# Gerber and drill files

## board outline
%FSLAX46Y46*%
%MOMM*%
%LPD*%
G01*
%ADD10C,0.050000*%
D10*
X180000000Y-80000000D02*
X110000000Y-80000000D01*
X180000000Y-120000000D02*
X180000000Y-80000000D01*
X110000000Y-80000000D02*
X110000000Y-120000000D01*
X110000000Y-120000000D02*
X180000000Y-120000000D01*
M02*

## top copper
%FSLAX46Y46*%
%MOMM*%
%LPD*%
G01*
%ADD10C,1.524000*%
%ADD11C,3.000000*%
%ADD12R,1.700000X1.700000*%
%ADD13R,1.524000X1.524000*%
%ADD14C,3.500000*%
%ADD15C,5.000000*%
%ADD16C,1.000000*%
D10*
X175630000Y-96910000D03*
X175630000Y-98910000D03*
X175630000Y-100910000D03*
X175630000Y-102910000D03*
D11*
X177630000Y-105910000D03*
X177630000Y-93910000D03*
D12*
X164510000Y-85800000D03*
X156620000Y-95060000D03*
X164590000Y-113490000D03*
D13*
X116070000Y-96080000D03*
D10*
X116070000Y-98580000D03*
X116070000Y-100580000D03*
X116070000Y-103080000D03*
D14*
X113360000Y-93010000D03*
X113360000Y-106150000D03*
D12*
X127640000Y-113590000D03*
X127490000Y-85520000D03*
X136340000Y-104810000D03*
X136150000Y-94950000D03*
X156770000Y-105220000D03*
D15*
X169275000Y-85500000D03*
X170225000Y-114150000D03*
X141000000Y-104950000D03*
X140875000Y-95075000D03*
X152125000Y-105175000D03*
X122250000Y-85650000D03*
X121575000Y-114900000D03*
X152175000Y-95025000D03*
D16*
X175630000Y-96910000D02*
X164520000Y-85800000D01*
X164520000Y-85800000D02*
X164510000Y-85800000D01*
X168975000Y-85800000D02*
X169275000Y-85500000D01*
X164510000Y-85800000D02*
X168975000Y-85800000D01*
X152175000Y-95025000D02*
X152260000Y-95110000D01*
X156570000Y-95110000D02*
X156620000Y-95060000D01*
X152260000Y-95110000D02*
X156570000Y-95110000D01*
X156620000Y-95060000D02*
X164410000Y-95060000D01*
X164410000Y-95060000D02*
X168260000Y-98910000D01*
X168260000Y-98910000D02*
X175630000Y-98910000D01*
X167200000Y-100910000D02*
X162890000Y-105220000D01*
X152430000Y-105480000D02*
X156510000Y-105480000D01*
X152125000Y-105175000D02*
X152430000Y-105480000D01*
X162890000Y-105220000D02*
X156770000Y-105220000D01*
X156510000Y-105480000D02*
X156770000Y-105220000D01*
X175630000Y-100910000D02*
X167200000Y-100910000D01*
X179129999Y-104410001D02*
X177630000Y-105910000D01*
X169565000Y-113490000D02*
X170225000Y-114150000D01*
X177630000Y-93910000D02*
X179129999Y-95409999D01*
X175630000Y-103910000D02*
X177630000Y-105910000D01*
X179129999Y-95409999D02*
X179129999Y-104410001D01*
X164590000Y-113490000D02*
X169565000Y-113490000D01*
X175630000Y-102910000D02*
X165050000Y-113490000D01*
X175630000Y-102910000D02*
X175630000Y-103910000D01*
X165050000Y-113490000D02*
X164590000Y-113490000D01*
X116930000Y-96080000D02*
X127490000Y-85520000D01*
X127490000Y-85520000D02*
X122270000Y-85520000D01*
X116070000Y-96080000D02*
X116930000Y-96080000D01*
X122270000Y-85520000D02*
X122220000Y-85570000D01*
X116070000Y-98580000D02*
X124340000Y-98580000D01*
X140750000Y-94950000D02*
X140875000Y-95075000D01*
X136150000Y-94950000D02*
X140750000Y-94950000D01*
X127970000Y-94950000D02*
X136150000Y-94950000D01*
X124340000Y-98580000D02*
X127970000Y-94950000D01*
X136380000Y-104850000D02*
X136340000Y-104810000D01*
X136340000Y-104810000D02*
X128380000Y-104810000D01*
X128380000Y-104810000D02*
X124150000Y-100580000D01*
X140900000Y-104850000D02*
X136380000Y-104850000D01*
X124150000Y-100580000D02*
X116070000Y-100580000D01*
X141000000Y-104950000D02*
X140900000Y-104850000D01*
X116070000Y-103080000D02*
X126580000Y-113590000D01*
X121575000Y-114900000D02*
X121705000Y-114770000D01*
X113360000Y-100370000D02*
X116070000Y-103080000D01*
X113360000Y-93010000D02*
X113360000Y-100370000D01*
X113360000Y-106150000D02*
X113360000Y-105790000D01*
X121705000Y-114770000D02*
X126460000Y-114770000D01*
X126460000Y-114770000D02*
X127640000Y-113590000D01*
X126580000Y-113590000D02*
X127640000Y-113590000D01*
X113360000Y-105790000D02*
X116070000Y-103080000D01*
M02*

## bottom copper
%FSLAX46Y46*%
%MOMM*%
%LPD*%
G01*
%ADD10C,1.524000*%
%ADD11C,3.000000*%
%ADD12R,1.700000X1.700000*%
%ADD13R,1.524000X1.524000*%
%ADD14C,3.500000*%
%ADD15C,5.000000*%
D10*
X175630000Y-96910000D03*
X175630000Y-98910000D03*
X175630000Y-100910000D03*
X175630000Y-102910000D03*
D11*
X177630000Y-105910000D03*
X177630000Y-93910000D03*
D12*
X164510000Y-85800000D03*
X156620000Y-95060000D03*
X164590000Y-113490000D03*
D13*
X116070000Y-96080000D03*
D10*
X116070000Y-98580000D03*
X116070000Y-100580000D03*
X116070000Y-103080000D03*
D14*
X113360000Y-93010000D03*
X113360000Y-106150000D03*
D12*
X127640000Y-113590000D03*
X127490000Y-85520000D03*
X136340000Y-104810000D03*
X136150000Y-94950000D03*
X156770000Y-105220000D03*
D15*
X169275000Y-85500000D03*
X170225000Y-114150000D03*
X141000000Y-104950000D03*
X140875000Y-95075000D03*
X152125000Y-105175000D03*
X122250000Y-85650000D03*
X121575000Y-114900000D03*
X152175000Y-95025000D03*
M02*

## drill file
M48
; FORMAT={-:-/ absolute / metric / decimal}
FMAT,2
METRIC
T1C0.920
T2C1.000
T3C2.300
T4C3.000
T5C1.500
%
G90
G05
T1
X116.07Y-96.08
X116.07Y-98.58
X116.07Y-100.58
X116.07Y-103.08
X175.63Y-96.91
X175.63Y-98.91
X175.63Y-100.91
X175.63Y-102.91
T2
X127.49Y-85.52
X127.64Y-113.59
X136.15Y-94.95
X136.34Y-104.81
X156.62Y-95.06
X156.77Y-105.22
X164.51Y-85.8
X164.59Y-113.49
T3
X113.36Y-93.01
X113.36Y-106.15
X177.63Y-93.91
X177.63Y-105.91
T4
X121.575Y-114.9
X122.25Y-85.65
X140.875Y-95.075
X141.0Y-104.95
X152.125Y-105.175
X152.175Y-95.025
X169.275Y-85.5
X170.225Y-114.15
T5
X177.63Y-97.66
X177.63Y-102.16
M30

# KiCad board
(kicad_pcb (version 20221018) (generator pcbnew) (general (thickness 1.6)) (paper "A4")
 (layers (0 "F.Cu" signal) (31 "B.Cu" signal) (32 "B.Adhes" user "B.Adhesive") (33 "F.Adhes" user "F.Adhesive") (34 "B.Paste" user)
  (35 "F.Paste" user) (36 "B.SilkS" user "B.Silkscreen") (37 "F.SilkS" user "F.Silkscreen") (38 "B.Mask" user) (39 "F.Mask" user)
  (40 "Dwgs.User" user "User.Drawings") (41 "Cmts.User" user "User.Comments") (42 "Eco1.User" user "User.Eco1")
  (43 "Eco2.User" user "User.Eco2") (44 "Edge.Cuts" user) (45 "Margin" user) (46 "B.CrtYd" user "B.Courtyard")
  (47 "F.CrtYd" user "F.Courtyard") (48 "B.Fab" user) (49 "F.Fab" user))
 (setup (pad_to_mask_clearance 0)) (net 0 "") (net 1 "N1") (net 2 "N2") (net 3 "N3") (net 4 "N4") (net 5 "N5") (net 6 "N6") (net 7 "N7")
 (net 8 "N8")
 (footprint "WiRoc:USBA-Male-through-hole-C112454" (layer "F.Cu") (at 177.63 99.91 90)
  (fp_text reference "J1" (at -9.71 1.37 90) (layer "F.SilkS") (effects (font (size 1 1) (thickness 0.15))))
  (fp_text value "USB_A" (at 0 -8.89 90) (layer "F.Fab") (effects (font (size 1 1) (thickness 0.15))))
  (pad "" np_thru_hole circle (at -2.25 0 90) (size 1.5 1.5) (drill 1.5) (layers "*.Cu" "*.Mask"))
  (pad "" np_thru_hole circle (at 2.25 0 90) (size 1.5 1.5) (drill 1.5) (layers "*.Cu" "*.Mask"))
  (pad "1" thru_hole circle (at 3 -2 90) (size 1.524 1.524) (drill 0.92) (layers "*.Cu" "*.Mask") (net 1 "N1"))
  (pad "2" thru_hole circle (at 1 -2 90) (size 1.524 1.524) (drill 0.92) (layers "*.Cu" "*.Mask") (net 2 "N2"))
  (pad "3" thru_hole circle (at -1 -2 90) (size 1.524 1.524) (drill 0.92) (layers "*.Cu" "*.Mask") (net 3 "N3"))
  (pad "4" thru_hole circle (at -3 -2 90) (size 1.524 1.524) (drill 0.92) (layers "*.Cu" "*.Mask") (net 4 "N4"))
  (pad "5" thru_hole circle (at -6 0 90) (size 3 3) (drill 2.3) (layers "*.Cu" "*.Mask") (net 4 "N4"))
  (pad "5" thru_hole circle (at 6 0 90) (size 3 3) (drill 2.3) (layers "*.Cu" "*.Mask") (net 4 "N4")))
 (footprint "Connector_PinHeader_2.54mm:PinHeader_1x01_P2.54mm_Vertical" (layer "F.Cu") (at 164.51 85.8 90)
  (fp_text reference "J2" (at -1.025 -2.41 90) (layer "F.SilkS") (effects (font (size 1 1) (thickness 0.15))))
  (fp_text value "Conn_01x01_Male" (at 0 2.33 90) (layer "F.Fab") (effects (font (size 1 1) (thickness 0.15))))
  (pad "1" thru_hole rect (at 0 0 90) (size 1.7 1.7) (drill 1) (layers "*.Cu" "*.Mask") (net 1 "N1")))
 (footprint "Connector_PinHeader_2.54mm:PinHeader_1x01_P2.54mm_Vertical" (layer "F.Cu") (at 156.62 95.06 90)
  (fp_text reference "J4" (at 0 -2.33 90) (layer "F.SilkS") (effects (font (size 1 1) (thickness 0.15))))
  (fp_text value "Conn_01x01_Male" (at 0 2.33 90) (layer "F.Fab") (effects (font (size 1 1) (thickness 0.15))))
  (pad "1" thru_hole rect (at 0 0 90) (size 1.7 1.7) (drill 1) (layers "*.Cu" "*.Mask") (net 2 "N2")))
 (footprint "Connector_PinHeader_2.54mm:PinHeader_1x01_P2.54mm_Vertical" (layer "F.Cu") (at 164.59 113.49 90)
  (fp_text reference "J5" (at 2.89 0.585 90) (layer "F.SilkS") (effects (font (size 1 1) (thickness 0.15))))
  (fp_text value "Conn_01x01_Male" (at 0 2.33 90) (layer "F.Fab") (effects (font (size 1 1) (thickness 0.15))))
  (pad "1" thru_hole rect (at 0 0 90) (size 1.7 1.7) (drill 1) (layers "*.Cu" "*.Mask") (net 4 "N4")))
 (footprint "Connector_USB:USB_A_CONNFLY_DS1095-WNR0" (layer "F.Cu") (at 116.07 96.08 -90)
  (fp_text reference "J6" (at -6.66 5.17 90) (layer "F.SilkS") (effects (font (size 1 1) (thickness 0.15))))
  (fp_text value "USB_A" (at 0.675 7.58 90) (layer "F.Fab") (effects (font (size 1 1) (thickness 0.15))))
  (pad "1" thru_hole rect (at 0 0 270) (size 1.524 1.524) (drill 0.92) (layers "*.Cu" "*.Mask") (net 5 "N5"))
  (pad "2" thru_hole circle (at 2.5 0 270) (size 1.524 1.524) (drill 0.92) (layers "*.Cu" "*.Mask") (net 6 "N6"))
  (pad "3" thru_hole circle (at 4.5 0 270) (size 1.524 1.524) (drill 0.92) (layers "*.Cu" "*.Mask") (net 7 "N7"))
  (pad "4" thru_hole circle (at 7 0 270) (size 1.524 1.524) (drill 0.92) (layers "*.Cu" "*.Mask") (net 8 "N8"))
  (pad "5" thru_hole circle (at -3.07 2.71 270) (size 3.5 3.5) (drill 2.3) (layers "*.Cu" "*.Mask") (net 8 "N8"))
  (pad "5" thru_hole circle (at 10.07 2.71 270) (size 3.5 3.5) (drill 2.3) (layers "*.Cu" "*.Mask") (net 8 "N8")))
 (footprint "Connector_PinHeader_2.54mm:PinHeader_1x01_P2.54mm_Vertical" (layer "F.Cu") (at 127.64 113.59 90)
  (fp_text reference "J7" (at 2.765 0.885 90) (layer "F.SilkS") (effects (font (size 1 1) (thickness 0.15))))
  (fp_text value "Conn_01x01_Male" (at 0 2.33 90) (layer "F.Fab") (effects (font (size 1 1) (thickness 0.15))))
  (pad "1" thru_hole rect (at 0 0 90) (size 1.7 1.7) (drill 1) (layers "*.Cu" "*.Mask") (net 8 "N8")))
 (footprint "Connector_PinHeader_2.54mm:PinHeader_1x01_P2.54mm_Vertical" (layer "F.Cu") (at 127.49 85.52 90)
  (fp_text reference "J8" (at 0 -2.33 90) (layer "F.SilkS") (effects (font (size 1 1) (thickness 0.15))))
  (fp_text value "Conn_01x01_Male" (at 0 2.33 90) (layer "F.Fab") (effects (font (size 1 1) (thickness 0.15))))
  (pad "1" thru_hole rect (at 0 0 90) (size 1.7 1.7) (drill 1) (layers "*.Cu" "*.Mask") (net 5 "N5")))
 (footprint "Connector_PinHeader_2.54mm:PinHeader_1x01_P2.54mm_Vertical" (layer "F.Cu") (at 136.34 104.81 90)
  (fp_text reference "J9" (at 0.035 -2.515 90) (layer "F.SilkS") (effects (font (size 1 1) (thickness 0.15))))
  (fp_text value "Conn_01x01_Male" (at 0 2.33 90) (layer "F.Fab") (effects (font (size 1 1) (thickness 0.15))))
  (pad "1" thru_hole rect (at 0 0 90) (size 1.7 1.7) (drill 1) (layers "*.Cu" "*.Mask") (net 7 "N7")))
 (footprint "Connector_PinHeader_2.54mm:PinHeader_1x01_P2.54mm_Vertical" (layer "F.Cu") (at 136.15 94.95 90)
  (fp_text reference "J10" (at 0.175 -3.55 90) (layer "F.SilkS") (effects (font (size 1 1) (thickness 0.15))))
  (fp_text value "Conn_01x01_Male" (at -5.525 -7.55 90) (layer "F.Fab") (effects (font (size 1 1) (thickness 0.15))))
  (pad "1" thru_hole rect (at 0 0 90) (size 1.7 1.7) (drill 1) (layers "*.Cu" "*.Mask") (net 6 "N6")))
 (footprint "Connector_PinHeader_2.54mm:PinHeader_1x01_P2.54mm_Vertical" (layer "F.Cu") (at 156.77 105.22 90)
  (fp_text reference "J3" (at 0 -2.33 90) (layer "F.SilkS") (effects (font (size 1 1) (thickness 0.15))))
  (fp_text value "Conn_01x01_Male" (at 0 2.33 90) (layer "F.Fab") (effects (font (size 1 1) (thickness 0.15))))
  (pad "1" thru_hole rect (at 0 0 90) (size 1.7 1.7) (drill 1) (layers "*.Cu" "*.Mask") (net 3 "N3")))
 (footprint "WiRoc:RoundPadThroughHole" (layer "F.Cu") (at 169.275 85.5)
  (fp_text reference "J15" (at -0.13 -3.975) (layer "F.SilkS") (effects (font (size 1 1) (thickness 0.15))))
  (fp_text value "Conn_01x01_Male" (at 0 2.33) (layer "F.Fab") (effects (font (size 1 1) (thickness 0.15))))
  (pad "1" thru_hole circle (at 0 0) (size 5 5) (drill 3) (layers "*.Cu" "*.Mask") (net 1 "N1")))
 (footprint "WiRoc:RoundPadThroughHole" (layer "F.Cu") (at 170.225 114.15)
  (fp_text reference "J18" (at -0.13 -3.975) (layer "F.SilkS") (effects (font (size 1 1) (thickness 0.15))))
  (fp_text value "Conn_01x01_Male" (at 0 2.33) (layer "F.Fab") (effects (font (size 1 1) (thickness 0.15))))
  (pad "1" thru_hole circle (at 0 0) (size 5 5) (drill 3) (layers "*.Cu" "*.Mask") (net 4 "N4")))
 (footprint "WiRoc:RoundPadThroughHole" (layer "F.Cu") (at 141 104.95)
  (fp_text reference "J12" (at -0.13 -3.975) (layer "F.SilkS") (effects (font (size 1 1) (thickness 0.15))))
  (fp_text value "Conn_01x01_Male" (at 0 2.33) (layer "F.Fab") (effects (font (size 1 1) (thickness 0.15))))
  (pad "1" thru_hole circle (at 0 0) (size 5 5) (drill 3) (layers "*.Cu" "*.Mask") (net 7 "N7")))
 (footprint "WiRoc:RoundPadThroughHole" (layer "F.Cu") (at 140.875 95.075)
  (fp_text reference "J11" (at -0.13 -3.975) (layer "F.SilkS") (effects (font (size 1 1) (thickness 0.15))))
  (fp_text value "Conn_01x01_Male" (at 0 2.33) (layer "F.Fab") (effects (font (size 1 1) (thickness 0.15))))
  (pad "1" thru_hole circle (at 0 0) (size 5 5) (drill 3) (layers "*.Cu" "*.Mask") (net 6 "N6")))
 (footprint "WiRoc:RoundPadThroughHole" (layer "F.Cu") (at 152.125 105.175)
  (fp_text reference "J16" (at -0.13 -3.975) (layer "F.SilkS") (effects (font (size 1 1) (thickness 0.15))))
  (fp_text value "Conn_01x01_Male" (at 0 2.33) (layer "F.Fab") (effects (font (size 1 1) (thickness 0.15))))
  (pad "1" thru_hole circle (at 0 0) (size 5 5) (drill 3) (layers "*.Cu" "*.Mask") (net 3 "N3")))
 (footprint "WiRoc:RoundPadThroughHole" (layer "F.Cu") (at 122.25 85.65)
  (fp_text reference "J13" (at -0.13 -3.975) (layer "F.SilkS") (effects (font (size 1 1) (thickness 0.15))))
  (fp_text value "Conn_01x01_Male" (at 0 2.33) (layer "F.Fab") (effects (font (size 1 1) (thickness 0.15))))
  (pad "1" thru_hole circle (at 0 0) (size 5 5) (drill 3) (layers "*.Cu" "*.Mask") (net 5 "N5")))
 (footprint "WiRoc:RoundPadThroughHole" (layer "F.Cu") (at 121.575 114.9)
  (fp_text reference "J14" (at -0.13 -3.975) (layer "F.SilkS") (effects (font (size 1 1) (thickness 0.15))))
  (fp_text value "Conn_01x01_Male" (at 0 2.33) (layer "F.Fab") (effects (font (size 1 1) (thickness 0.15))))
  (pad "1" thru_hole circle (at 0 0) (size 5 5) (drill 3) (layers "*.Cu" "*.Mask") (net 8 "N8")))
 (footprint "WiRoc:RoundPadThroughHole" (layer "F.Cu") (at 152.175 95.025)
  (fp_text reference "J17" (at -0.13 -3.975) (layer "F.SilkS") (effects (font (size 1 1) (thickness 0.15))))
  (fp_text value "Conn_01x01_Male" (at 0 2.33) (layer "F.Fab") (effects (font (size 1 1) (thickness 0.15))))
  (pad "1" thru_hole circle (at 0 0) (size 5 5) (drill 3) (layers "*.Cu" "*.Mask") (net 2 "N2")))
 (gr_line (start 180 80) (end 110 80) (stroke (width 0.05) (type solid)) (layer "Edge.Cuts"))
 (gr_line (start 180 120) (end 180 80) (stroke (width 0.05) (type solid)) (layer "Edge.Cuts"))
 (gr_line (start 110 80) (end 110 120) (stroke (width 0.05) (type solid)) (layer "Edge.Cuts"))
 (gr_line (start 110 120) (end 180 120) (stroke (width 0.05) (type solid)) (layer "Edge.Cuts"))
 (segment (start 175.63 96.91) (end 164.52 85.8) (width 1) (layer "F.Cu") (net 1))
 (segment (start 164.52 85.8) (end 164.51 85.8) (width 1) (layer "F.Cu") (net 1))
 (segment (start 168.975 85.8) (end 169.275 85.5) (width 1) (layer "F.Cu") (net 1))
 (segment (start 164.51 85.8) (end 168.975 85.8) (width 1) (layer "F.Cu") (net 1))
 (segment (start 152.175 95.025) (end 152.26 95.11) (width 1) (layer "F.Cu") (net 2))
 (segment (start 156.57 95.11) (end 156.62 95.06) (width 1) (layer "F.Cu") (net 2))
 (segment (start 152.26 95.11) (end 156.57 95.11) (width 1) (layer "F.Cu") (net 2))
 (segment (start 156.62 95.06) (end 164.41 95.06) (width 1) (layer "F.Cu") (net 2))
 (segment (start 164.41 95.06) (end 168.26 98.91) (width 1) (layer "F.Cu") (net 2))
 (segment (start 168.26 98.91) (end 175.63 98.91) (width 1) (layer "F.Cu") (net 2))
 (segment (start 167.2 100.91) (end 162.89 105.22) (width 1) (layer "F.Cu") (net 3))
 (segment (start 152.43 105.48) (end 156.51 105.48) (width 1) (layer "F.Cu") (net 3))
 (segment (start 152.125 105.175) (end 152.43 105.48) (width 1) (layer "F.Cu") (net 3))
 (segment (start 162.89 105.22) (end 156.77 105.22) (width 1) (layer "F.Cu") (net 3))
 (segment (start 156.51 105.48) (end 156.77 105.22) (width 1) (layer "F.Cu") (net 3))
 (segment (start 175.63 100.91) (end 167.2 100.91) (width 1) (layer "F.Cu") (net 3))
 (segment (start 179.129999 104.410001) (end 177.63 105.91) (width 1) (layer "F.Cu") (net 4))
 (segment (start 169.565 113.49) (end 170.225 114.15) (width 1) (layer "F.Cu") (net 4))
 (segment (start 177.63 93.91) (end 179.129999 95.409999) (width 1) (layer "F.Cu") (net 4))
 (segment (start 175.63 103.91) (end 177.63 105.91) (width 1) (layer "F.Cu") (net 4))
 (segment (start 179.129999 95.409999) (end 179.129999 104.410001) (width 1) (layer "F.Cu") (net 4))
 (segment (start 164.59 113.49) (end 169.565 113.49) (width 1) (layer "F.Cu") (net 4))
 (segment (start 175.63 102.91) (end 165.05 113.49) (width 1) (layer "F.Cu") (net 4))
 (segment (start 175.63 102.91) (end 175.63 103.91) (width 1) (layer "F.Cu") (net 4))
 (segment (start 165.05 113.49) (end 164.59 113.49) (width 1) (layer "F.Cu") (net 4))
 (segment (start 116.93 96.08) (end 127.49 85.52) (width 1) (layer "F.Cu") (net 5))
 (segment (start 127.49 85.52) (end 122.27 85.52) (width 1) (layer "F.Cu") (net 5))
 (segment (start 116.07 96.08) (end 116.93 96.08) (width 1) (layer "F.Cu") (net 5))
 (segment (start 122.27 85.52) (end 122.22 85.57) (width 1) (layer "F.Cu") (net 5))
 (segment (start 116.07 98.58) (end 124.34 98.58) (width 1) (layer "F.Cu") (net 6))
 (segment (start 140.75 94.95) (end 140.875 95.075) (width 1) (layer "F.Cu") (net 6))
 (segment (start 136.15 94.95) (end 140.75 94.95) (width 1) (layer "F.Cu") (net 6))
 (segment (start 127.97 94.95) (end 136.15 94.95) (width 1) (layer "F.Cu") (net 6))
 (segment (start 124.34 98.58) (end 127.97 94.95) (width 1) (layer "F.Cu") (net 6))
 (segment (start 136.38 104.85) (end 136.34 104.81) (width 1) (layer "F.Cu") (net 7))
 (segment (start 136.34 104.81) (end 128.38 104.81) (width 1) (layer "F.Cu") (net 7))
 (segment (start 128.38 104.81) (end 124.15 100.58) (width 1) (layer "F.Cu") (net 7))
 (segment (start 140.9 104.85) (end 136.38 104.85) (width 1) (layer "F.Cu") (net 7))
 (segment (start 124.15 100.58) (end 116.07 100.58) (width 1) (layer "F.Cu") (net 7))
 (segment (start 141 104.95) (end 140.9 104.85) (width 1) (layer "F.Cu") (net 7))
 (segment (start 116.07 103.08) (end 126.58 113.59) (width 1) (layer "F.Cu") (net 8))
 (segment (start 121.575 114.9) (end 121.705 114.77) (width 1) (layer "F.Cu") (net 8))
 (segment (start 113.36 100.37) (end 116.07 103.08) (width 1) (layer "F.Cu") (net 8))
 (segment (start 113.36 93.01) (end 113.36 100.37) (width 1) (layer "F.Cu") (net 8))
 (segment (start 113.36 106.15) (end 113.36 105.79) (width 1) (layer "F.Cu") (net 8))
 (segment (start 121.705 114.77) (end 126.46 114.77) (width 1) (layer "F.Cu") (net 8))
 (segment (start 126.46 114.77) (end 127.64 113.59) (width 1) (layer "F.Cu") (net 8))
 (segment (start 126.58 113.59) (end 127.64 113.59) (width 1) (layer "F.Cu") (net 8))
 (segment (start 113.36 105.79) (end 116.07 103.08) (width 1) (layer "F.Cu") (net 8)))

